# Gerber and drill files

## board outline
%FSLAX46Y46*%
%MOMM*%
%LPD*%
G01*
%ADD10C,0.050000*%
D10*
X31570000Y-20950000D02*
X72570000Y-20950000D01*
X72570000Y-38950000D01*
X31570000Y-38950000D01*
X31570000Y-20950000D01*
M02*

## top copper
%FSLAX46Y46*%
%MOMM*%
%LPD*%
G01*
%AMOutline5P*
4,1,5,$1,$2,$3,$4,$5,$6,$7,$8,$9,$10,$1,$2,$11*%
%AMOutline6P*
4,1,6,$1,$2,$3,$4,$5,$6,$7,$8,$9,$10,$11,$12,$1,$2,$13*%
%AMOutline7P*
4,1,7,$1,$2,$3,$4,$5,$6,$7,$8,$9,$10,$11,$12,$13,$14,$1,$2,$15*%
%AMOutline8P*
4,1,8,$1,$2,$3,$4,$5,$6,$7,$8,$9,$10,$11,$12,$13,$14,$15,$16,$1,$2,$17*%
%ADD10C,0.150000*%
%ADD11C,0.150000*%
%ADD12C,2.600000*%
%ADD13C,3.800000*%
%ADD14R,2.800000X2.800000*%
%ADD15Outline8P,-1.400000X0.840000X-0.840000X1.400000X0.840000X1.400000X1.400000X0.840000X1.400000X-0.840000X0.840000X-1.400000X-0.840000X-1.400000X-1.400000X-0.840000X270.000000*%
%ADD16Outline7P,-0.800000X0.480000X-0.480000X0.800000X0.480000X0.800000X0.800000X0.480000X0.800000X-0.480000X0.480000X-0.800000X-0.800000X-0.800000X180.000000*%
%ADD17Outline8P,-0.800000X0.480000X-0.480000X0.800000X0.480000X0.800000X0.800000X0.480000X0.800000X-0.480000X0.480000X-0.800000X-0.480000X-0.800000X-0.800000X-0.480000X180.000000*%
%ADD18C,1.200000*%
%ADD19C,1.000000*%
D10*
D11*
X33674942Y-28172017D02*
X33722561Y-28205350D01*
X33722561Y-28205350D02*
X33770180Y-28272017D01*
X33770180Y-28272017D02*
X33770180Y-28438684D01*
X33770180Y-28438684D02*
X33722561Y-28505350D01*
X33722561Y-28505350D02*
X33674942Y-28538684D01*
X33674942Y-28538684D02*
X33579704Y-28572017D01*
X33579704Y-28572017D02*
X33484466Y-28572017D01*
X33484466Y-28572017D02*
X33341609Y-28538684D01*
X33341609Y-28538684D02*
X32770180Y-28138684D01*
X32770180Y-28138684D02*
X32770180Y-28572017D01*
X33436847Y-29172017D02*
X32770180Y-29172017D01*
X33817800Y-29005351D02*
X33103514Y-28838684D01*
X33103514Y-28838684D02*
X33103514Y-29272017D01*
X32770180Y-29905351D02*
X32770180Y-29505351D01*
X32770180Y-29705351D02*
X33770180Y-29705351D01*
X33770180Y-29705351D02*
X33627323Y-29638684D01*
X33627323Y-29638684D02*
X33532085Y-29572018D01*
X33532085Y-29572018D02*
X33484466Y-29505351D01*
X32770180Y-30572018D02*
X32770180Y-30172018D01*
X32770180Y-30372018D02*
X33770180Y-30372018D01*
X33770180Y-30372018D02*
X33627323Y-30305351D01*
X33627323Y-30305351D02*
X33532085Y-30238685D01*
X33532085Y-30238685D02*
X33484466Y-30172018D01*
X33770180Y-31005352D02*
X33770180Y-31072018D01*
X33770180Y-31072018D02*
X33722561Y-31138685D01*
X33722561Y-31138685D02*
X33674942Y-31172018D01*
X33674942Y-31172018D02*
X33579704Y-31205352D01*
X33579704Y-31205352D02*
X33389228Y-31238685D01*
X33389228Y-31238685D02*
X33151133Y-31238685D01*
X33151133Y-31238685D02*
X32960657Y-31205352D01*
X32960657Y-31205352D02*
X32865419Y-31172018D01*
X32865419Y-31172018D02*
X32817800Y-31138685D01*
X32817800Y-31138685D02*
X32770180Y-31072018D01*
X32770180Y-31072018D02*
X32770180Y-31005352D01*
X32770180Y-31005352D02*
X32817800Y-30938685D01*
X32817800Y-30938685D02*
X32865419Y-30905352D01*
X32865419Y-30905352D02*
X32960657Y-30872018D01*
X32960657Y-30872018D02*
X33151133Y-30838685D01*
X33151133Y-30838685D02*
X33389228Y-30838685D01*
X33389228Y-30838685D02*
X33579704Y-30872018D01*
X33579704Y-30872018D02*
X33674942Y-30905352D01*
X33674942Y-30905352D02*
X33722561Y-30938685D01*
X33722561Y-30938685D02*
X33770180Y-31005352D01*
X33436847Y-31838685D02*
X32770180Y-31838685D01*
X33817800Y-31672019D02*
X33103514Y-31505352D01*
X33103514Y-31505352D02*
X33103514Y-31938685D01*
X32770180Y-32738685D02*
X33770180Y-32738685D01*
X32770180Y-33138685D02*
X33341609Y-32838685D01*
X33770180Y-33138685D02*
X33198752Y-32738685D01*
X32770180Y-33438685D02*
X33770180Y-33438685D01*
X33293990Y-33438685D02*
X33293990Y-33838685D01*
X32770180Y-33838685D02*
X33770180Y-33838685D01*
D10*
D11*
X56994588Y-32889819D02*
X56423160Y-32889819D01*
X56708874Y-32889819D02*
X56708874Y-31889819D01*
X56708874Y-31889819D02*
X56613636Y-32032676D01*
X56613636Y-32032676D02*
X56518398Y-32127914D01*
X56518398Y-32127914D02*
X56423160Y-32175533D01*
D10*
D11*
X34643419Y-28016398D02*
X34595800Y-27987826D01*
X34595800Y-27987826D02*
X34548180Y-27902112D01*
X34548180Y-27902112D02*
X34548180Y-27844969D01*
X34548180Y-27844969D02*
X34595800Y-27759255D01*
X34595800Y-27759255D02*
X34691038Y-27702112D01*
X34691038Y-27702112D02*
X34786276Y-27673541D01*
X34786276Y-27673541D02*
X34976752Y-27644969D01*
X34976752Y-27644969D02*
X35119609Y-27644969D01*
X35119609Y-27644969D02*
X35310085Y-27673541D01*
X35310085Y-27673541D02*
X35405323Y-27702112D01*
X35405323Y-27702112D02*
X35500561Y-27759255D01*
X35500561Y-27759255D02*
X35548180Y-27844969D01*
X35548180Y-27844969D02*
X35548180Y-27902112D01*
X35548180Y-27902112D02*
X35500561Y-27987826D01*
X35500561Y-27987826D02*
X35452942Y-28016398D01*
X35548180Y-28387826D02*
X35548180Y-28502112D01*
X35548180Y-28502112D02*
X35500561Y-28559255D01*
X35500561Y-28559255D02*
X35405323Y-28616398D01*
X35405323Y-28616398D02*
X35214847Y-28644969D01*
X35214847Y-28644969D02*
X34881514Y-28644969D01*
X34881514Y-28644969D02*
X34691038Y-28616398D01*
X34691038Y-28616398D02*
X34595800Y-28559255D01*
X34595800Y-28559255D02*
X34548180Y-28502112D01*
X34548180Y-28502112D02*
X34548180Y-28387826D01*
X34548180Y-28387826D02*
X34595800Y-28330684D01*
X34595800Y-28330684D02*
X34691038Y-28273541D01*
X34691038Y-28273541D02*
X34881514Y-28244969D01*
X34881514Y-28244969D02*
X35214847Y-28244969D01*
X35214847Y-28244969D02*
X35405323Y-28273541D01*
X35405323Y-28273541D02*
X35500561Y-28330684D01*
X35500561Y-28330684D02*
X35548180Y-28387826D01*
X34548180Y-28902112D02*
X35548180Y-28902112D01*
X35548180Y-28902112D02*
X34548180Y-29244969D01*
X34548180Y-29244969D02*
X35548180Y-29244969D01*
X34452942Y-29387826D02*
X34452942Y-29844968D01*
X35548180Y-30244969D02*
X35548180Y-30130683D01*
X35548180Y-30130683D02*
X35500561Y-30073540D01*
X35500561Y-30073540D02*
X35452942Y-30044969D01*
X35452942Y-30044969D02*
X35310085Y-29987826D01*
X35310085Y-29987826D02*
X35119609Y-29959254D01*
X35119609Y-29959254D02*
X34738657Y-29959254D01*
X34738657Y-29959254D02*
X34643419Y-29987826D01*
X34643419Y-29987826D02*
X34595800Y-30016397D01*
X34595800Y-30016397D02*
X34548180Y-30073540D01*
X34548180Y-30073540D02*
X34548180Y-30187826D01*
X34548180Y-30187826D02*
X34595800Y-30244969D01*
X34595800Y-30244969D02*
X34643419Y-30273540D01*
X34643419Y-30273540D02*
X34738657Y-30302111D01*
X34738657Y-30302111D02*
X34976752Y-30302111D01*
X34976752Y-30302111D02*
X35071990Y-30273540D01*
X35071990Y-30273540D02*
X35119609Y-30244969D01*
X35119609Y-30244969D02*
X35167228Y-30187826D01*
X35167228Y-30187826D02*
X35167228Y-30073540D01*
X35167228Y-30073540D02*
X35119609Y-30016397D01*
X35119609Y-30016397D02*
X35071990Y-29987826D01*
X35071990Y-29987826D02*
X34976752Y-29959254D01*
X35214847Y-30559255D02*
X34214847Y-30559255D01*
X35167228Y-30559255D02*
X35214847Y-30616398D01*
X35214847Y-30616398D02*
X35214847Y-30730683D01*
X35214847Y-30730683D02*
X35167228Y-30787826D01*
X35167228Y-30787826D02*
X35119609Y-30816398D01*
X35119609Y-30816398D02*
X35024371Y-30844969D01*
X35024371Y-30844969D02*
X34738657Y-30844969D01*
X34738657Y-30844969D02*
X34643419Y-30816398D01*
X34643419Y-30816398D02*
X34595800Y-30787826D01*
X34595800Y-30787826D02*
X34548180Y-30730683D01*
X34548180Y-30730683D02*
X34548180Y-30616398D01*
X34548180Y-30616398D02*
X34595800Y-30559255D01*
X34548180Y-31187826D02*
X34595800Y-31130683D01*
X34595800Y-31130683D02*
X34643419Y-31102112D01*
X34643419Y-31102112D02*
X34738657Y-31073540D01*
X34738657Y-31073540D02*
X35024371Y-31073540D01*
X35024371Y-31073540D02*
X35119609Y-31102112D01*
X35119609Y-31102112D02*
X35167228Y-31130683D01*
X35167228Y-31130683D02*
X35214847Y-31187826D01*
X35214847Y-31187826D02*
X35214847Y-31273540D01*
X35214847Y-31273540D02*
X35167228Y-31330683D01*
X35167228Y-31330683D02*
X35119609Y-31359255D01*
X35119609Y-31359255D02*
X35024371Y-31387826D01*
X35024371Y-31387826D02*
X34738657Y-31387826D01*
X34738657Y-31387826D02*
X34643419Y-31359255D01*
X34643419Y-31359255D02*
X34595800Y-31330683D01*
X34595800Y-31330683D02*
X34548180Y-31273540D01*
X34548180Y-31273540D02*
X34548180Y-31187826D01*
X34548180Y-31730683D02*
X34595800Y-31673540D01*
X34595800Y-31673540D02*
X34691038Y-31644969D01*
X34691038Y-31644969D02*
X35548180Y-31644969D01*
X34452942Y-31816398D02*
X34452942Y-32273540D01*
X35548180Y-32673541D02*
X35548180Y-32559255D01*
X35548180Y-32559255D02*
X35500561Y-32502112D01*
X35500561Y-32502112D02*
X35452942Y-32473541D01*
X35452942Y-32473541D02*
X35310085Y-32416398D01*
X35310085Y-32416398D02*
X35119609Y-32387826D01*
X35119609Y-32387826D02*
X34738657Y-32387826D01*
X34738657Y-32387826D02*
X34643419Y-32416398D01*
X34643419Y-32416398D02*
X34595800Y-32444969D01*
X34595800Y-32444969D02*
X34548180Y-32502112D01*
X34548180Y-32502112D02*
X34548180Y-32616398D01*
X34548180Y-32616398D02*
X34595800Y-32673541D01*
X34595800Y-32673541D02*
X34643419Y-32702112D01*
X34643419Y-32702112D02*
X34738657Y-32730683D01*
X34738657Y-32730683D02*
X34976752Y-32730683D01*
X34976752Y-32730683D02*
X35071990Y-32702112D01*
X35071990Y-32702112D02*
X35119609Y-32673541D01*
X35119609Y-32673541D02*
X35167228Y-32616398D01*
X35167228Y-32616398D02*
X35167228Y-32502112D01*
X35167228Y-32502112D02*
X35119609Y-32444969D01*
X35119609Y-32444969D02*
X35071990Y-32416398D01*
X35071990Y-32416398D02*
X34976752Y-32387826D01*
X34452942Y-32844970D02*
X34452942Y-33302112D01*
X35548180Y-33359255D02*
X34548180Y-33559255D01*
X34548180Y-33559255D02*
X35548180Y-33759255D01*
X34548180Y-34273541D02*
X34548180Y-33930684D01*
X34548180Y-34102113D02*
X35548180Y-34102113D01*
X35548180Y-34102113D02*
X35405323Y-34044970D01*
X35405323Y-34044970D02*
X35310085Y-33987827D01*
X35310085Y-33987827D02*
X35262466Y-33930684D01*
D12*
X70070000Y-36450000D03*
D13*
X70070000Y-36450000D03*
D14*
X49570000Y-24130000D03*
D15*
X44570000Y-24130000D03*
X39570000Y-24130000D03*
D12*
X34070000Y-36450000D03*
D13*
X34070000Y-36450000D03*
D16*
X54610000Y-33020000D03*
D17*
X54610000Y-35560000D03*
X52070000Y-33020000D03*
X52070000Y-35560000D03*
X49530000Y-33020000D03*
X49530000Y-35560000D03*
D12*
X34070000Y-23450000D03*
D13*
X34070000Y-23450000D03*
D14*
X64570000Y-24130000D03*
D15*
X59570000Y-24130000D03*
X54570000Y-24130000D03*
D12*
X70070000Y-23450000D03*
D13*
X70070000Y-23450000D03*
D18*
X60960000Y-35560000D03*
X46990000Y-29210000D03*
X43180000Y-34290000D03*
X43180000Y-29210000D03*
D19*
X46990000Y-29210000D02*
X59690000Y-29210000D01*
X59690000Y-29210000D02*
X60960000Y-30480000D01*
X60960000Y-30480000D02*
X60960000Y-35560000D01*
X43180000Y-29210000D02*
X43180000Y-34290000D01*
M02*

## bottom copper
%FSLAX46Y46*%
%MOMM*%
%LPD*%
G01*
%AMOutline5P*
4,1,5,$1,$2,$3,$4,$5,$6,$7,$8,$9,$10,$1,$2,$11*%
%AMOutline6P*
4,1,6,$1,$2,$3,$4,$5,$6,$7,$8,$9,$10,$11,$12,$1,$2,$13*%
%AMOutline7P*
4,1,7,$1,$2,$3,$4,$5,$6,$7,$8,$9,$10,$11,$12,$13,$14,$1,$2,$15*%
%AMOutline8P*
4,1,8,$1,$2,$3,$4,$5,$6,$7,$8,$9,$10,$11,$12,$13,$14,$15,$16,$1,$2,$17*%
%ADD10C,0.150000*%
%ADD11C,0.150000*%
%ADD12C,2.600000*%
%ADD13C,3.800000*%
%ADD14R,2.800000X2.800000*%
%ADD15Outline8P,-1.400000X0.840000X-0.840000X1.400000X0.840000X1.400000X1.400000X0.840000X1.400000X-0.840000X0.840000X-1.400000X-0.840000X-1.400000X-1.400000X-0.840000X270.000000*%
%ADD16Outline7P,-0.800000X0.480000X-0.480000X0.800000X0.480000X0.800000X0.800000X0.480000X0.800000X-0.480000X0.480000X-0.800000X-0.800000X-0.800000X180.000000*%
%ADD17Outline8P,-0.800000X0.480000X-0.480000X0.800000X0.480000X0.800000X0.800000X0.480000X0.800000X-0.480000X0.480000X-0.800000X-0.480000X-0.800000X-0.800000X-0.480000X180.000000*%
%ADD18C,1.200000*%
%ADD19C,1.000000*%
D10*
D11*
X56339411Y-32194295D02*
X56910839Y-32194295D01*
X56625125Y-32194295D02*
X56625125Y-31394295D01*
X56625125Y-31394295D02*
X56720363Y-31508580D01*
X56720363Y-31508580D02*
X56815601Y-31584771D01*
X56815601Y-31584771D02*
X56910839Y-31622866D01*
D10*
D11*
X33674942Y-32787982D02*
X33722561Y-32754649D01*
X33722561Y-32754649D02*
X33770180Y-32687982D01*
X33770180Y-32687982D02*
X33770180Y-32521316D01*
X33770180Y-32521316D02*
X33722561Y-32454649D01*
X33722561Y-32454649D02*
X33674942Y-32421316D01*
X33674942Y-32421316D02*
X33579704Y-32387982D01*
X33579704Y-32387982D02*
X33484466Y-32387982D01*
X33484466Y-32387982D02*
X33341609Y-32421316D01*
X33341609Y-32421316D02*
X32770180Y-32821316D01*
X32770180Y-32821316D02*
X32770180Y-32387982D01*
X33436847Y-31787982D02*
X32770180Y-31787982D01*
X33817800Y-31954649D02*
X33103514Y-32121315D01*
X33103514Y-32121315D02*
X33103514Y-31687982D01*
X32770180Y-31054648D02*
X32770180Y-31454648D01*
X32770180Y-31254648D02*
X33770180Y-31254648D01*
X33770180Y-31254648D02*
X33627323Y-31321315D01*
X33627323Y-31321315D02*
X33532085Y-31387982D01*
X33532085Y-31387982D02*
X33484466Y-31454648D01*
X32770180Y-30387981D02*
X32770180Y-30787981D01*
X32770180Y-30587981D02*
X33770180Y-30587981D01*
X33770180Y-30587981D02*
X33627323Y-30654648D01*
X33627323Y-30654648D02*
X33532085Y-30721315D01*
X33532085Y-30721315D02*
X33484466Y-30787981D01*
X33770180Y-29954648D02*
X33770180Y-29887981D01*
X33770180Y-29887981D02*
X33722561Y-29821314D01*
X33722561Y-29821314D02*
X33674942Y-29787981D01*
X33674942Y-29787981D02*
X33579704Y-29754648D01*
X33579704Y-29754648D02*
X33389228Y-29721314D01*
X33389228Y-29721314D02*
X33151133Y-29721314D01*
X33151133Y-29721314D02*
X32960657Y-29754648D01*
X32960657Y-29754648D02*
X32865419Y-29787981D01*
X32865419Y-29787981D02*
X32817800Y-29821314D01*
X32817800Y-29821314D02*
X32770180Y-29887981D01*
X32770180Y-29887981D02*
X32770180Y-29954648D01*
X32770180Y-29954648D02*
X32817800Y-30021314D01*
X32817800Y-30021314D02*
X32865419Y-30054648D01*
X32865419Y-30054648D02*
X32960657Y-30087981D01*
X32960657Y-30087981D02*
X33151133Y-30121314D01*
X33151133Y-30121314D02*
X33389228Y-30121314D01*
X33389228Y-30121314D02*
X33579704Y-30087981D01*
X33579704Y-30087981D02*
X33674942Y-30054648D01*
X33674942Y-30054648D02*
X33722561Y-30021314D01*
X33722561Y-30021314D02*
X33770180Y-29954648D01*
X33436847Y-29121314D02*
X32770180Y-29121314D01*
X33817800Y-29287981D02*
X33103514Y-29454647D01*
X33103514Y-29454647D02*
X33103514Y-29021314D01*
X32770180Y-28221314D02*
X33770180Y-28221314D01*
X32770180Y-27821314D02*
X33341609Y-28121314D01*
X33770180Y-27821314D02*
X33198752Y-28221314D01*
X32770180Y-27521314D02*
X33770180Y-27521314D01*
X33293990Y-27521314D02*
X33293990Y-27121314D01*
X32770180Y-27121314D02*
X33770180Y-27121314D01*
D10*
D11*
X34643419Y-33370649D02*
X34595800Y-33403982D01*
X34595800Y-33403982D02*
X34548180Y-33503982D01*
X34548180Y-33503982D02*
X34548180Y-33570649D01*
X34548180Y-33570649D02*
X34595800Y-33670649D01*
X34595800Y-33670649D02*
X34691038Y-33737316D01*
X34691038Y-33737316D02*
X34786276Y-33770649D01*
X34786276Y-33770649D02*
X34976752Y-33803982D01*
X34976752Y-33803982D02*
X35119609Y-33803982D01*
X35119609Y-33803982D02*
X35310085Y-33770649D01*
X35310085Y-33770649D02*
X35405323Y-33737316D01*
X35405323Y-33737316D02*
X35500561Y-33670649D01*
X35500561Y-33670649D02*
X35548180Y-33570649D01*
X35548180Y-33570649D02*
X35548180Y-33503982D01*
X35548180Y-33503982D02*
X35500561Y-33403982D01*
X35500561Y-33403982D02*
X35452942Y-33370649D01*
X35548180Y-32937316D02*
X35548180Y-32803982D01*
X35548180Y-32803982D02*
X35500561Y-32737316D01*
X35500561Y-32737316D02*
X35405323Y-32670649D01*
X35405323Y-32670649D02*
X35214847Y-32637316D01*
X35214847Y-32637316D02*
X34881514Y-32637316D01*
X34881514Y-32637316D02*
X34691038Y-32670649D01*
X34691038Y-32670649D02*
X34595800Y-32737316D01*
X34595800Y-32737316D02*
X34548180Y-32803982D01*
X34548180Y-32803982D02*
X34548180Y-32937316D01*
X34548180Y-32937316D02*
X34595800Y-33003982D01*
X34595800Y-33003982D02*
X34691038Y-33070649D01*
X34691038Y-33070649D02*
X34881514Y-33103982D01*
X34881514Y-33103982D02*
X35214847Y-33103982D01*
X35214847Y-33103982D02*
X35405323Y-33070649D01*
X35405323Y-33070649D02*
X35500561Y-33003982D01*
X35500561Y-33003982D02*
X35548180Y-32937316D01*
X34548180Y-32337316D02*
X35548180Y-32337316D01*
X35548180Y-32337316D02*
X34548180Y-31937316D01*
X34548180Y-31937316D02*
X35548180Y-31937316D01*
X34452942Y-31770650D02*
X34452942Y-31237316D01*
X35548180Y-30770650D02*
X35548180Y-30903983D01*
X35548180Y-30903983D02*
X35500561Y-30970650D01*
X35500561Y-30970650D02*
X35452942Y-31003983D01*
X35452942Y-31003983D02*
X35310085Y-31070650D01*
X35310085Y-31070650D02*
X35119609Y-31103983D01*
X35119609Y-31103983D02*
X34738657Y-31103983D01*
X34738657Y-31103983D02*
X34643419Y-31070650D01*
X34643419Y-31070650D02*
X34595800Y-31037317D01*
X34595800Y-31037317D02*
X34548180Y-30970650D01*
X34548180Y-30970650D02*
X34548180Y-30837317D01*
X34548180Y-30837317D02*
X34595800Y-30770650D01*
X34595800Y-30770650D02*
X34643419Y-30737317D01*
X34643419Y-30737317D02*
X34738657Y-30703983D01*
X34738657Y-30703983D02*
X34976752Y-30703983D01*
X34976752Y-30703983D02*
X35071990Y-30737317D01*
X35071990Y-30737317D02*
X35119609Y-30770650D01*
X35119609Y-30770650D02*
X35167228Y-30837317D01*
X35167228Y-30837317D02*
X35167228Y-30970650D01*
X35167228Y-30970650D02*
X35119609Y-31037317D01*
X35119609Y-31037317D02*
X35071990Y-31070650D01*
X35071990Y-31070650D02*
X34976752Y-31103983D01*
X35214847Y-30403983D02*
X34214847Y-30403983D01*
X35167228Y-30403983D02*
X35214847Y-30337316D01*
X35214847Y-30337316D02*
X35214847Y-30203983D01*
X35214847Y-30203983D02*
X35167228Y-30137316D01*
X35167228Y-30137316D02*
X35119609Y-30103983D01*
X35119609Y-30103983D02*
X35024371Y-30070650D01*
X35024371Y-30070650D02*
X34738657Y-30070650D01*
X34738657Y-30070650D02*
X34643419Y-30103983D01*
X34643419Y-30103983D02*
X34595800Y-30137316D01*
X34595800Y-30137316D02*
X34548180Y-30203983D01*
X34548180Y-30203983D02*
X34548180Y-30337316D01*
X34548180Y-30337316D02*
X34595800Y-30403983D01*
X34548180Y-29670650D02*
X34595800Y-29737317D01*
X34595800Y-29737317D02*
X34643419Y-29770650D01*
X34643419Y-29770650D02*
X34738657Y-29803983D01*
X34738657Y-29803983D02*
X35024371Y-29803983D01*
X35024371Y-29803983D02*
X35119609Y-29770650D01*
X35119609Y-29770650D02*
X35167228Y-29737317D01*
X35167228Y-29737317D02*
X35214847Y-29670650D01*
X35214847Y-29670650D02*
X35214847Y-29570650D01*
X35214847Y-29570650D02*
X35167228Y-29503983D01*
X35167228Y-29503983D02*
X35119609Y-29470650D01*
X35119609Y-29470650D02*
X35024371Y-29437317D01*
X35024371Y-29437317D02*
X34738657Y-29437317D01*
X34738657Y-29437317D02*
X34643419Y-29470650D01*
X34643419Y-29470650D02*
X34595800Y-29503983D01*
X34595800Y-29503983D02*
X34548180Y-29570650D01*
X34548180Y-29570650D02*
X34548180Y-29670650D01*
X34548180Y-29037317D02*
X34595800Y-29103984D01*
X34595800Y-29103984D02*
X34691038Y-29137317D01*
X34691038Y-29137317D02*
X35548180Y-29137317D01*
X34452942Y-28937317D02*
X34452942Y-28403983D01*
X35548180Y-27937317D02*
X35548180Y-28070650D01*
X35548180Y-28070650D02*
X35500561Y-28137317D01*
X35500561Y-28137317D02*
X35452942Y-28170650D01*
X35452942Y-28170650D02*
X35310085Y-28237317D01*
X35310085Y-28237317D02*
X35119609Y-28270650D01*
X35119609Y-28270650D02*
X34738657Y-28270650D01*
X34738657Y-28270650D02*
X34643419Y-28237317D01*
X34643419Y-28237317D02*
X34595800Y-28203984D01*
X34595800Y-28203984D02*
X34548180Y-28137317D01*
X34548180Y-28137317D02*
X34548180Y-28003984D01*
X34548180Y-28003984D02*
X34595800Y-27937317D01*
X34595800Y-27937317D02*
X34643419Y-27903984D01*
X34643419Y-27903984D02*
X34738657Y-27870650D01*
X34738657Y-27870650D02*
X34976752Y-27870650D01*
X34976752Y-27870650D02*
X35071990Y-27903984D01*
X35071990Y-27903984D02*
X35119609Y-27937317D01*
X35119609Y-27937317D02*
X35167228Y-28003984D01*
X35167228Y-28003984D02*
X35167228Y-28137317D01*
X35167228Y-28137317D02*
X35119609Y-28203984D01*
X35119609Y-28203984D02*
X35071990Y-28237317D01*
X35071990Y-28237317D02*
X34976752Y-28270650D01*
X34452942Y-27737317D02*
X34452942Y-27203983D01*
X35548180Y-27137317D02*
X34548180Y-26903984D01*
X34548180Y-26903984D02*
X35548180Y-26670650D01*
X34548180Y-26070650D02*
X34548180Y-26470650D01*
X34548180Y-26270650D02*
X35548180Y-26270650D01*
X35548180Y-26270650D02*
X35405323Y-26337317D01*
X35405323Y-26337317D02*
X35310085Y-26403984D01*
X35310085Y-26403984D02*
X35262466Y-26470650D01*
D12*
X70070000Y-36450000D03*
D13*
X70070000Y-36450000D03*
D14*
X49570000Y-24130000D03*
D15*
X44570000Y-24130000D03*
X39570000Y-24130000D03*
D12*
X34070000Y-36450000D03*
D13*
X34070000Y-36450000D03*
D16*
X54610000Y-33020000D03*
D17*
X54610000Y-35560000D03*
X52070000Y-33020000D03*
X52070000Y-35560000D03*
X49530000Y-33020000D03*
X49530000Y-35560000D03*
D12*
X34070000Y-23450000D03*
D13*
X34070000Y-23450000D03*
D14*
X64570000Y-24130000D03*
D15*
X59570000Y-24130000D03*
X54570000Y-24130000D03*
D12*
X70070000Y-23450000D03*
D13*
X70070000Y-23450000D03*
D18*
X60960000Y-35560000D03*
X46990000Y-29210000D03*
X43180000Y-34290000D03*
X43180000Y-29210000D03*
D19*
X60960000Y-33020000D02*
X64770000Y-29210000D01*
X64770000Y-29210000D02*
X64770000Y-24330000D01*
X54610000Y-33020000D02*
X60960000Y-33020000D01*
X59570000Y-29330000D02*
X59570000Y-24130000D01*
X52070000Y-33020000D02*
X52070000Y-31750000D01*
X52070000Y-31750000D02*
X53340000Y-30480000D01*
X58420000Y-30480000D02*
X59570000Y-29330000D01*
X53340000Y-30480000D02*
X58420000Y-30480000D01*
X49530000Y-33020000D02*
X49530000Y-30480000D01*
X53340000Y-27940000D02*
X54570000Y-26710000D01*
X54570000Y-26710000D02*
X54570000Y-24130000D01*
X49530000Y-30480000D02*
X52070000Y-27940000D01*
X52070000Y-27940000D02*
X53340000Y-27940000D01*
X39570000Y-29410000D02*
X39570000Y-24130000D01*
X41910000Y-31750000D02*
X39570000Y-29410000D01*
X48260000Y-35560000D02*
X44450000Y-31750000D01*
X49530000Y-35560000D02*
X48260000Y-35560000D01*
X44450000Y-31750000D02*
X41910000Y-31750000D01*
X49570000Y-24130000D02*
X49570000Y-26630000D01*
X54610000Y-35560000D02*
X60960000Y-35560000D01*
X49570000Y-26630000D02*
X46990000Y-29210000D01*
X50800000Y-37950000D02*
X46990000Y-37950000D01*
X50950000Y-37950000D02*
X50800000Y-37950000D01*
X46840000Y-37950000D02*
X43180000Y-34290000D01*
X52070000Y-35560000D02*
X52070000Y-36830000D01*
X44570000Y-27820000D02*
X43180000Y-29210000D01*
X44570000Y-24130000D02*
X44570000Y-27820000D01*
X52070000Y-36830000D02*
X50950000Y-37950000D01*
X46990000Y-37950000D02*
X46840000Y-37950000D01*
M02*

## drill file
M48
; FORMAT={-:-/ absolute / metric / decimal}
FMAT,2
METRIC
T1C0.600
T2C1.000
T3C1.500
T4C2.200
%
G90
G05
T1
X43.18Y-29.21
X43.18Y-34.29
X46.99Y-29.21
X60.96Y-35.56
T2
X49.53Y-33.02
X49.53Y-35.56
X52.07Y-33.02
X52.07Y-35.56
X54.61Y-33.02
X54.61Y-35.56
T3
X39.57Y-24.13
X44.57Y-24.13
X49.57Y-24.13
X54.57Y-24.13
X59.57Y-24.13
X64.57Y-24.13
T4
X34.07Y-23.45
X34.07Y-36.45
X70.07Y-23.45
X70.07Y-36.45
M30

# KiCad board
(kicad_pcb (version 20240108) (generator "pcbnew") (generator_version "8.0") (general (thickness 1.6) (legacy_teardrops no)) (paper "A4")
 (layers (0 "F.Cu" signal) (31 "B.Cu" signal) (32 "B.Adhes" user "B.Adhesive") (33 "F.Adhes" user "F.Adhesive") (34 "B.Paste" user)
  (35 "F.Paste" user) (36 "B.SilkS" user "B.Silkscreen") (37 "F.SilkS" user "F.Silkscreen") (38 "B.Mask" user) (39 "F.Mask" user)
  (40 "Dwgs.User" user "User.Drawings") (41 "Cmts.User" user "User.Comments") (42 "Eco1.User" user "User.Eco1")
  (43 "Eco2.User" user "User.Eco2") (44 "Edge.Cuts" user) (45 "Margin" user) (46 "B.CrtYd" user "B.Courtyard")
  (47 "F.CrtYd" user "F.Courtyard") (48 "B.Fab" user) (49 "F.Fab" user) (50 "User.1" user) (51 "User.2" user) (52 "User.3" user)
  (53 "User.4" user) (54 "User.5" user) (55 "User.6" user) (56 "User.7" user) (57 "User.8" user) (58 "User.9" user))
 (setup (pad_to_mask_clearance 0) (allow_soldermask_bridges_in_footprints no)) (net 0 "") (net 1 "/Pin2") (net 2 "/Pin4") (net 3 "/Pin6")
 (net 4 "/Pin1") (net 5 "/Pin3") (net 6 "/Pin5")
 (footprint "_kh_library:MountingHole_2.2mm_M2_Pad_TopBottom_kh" (layer "F.Cu") (at 70.07 36.45)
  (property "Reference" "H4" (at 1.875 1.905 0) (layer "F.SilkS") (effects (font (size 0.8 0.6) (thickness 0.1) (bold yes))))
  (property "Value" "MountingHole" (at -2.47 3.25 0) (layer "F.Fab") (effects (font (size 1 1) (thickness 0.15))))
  (pad "1" thru_hole circle (at 0 0) (size 2.6 2.6) (drill 2.2) (layers "*.Cu" "*.Mask") (remove_unused_layers no))
  (pad "1" connect circle (at 0 0) (size 3.8 3.8) (layers "F.Cu" "F.Mask"))
  (pad "1" connect circle (at 0 0) (size 3.8 3.8) (layers "B.Cu" "B.Mask")))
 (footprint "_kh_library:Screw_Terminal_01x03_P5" (layer "F.Cu") (at 49.57 24.13 -90)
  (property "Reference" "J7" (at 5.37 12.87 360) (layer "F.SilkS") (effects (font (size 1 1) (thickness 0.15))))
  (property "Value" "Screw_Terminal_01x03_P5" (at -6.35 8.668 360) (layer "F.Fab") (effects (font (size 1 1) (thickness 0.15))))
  (pad "1" thru_hole rect (at 0 0 270) (size 2.8 2.8) (drill 1.5) (layers "*.Cu" "*.Mask") (remove_unused_layers no) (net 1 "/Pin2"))
  (pad "2" thru_hole roundrect (at 0 5 270) (size 2.8 2.8) (drill 1.5) (layers "*.Cu" "*.Mask") (remove_unused_layers no)
   (roundrect_rratio 0) (chamfer_ratio 0.2) (chamfer top_left top_right bottom_left bottom_right) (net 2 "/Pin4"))
  (pad "3" thru_hole roundrect (at 0 10 270) (size 2.8 2.8) (drill 1.5) (layers "*.Cu" "*.Mask") (remove_unused_layers no)
   (roundrect_rratio 0) (chamfer_ratio 0.2) (chamfer top_left top_right bottom_left bottom_right) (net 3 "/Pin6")))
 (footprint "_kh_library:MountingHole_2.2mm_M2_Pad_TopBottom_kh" (layer "F.Cu") (at 34.07 36.45)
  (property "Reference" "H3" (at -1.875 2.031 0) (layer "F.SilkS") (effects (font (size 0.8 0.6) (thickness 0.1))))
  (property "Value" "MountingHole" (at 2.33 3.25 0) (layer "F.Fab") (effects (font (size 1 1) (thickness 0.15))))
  (pad "1" thru_hole circle (at 0 0) (size 2.6 2.6) (drill 2.2) (layers "*.Cu" "*.Mask") (remove_unused_layers no))
  (pad "1" connect circle (at 0 0) (size 3.8 3.8) (layers "F.Cu" "F.Mask"))
  (pad "1" connect circle (at 0 0) (size 3.8 3.8) (layers "B.Cu" "B.Mask")))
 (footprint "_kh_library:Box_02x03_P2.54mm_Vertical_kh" (layer "F.Cu") (at 54.61 33.02 180)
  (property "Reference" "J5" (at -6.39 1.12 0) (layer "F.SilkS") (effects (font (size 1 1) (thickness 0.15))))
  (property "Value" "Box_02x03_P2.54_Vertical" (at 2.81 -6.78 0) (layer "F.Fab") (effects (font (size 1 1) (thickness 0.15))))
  (pad "1" thru_hole roundrect (at 0 0 180) (size 1.6 1.6) (drill 1) (layers "*.Cu" "*.Mask") (remove_unused_layers no) (roundrect_rratio 0)
   (chamfer_ratio 0.2) (chamfer top_left top_right bottom_right) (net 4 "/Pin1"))
  (pad "2" thru_hole roundrect (at 0 -2.54 180) (size 1.6 1.6) (drill 1) (layers "*.Cu" "*.Mask") (remove_unused_layers no)
   (roundrect_rratio 0) (chamfer_ratio 0.2) (chamfer top_left top_right bottom_left bottom_right) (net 1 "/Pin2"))
  (pad "3" thru_hole roundrect (at 2.54 0 180) (size 1.6 1.6) (drill 1) (layers "*.Cu" "*.Mask") (remove_unused_layers no)
   (roundrect_rratio 0) (chamfer_ratio 0.2) (chamfer top_left top_right bottom_left bottom_right) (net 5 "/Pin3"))
  (pad "4" thru_hole roundrect (at 2.54 -2.54 180) (size 1.6 1.6) (drill 1) (layers "*.Cu" "*.Mask") (remove_unused_layers no)
   (roundrect_rratio 0) (chamfer_ratio 0.2) (chamfer top_left top_right bottom_left bottom_right) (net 2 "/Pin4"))
  (pad "5" thru_hole roundrect (at 5.08 0 180) (size 1.6 1.6) (drill 1) (layers "*.Cu" "*.Mask") (remove_unused_layers no)
   (roundrect_rratio 0) (chamfer_ratio 0.2) (chamfer top_left top_right bottom_left bottom_right) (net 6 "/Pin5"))
  (pad "6" thru_hole roundrect (at 5.08 -2.54 180) (size 1.6 1.6) (drill 1) (layers "*.Cu" "*.Mask") (remove_unused_layers no)
   (roundrect_rratio 0) (chamfer_ratio 0.2) (chamfer top_left top_right bottom_left bottom_right) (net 3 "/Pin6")))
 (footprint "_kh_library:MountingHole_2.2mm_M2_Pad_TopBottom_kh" (layer "F.Cu") (at 34.07 23.45)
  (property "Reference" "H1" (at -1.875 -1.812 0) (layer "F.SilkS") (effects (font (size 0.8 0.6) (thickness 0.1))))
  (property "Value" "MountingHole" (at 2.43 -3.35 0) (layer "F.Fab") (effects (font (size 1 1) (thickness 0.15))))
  (pad "1" thru_hole circle (at 0 0) (size 2.6 2.6) (drill 2.2) (layers "*.Cu" "*.Mask") (remove_unused_layers no))
  (pad "1" connect circle (at 0 0) (size 3.8 3.8) (layers "F.Cu" "F.Mask"))
  (pad "1" connect circle (at 0 0) (size 3.8 3.8) (layers "B.Cu" "B.Mask")))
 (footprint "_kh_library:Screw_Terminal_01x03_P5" (layer "F.Cu") (at 64.57 24.13 -90)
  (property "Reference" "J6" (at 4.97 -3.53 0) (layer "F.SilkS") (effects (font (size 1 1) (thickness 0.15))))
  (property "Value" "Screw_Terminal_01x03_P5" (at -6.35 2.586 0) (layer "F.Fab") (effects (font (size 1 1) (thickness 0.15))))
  (pad "1" thru_hole rect (at 0 0 270) (size 2.8 2.8) (drill 1.5) (layers "*.Cu" "*.Mask") (remove_unused_layers no) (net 4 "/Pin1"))
  (pad "2" thru_hole roundrect (at 0 5 270) (size 2.8 2.8) (drill 1.5) (layers "*.Cu" "*.Mask") (remove_unused_layers no)
   (roundrect_rratio 0) (chamfer_ratio 0.2) (chamfer top_left top_right bottom_left bottom_right) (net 5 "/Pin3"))
  (pad "3" thru_hole roundrect (at 0 10 270) (size 2.8 2.8) (drill 1.5) (layers "*.Cu" "*.Mask") (remove_unused_layers no)
   (roundrect_rratio 0) (chamfer_ratio 0.2) (chamfer top_left top_right bottom_left bottom_right) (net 6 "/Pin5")))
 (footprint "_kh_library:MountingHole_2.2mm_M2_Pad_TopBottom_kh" (layer "F.Cu") (at 70.07 23.45)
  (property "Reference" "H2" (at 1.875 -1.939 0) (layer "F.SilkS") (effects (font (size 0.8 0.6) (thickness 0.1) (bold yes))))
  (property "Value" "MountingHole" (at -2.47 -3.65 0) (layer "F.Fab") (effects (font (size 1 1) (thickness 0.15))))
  (pad "1" thru_hole circle (at 0 0) (size 2.6 2.6) (drill 2.2) (layers "*.Cu" "*.Mask") (remove_unused_layers no))
  (pad "1" connect circle (at 0 0) (size 3.8 3.8) (layers "F.Cu" "F.Mask"))
  (pad "1" connect circle (at 0 0) (size 3.8 3.8) (layers "B.Cu" "B.Mask")))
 (gr_rect (start 31.57 20.95) (end 72.57 38.95) (stroke (width 0.05) (type default)) (fill none) (layer "Edge.Cuts"))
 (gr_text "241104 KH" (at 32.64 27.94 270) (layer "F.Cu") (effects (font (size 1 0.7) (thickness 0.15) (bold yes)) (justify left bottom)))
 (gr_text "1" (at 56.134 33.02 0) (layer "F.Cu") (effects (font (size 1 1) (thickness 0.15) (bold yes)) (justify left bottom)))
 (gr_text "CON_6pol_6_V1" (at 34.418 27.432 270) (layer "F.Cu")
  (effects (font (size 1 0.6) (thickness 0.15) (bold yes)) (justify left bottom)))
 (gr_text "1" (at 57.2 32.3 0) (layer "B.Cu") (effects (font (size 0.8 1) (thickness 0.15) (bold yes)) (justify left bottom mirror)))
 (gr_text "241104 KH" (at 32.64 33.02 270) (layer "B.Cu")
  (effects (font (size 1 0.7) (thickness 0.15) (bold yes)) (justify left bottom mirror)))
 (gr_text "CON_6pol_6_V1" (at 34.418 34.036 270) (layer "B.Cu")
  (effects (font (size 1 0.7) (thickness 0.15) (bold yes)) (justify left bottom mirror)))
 (segment (start 60.96 33.02) (end 64.77 29.21) (width 1) (layer "B.Cu") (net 4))
 (segment (start 64.77 29.21) (end 64.77 24.33) (width 1) (layer "B.Cu") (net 4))
 (segment (start 54.61 33.02) (end 60.96 33.02) (width 1) (layer "B.Cu") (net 4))
 (segment (start 59.57 29.33) (end 59.57 24.13) (width 1) (layer "B.Cu") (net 5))
 (segment (start 52.07 33.02) (end 52.07 31.75) (width 1) (layer "B.Cu") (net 5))
 (segment (start 52.07 31.75) (end 53.34 30.48) (width 1) (layer "B.Cu") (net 5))
 (segment (start 58.42 30.48) (end 59.57 29.33) (width 1) (layer "B.Cu") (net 5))
 (segment (start 53.34 30.48) (end 58.42 30.48) (width 1) (layer "B.Cu") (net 5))
 (segment (start 49.53 33.02) (end 49.53 30.48) (width 1) (layer "B.Cu") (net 6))
 (segment (start 53.34 27.94) (end 54.57 26.71) (width 1) (layer "B.Cu") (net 6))
 (segment (start 54.57 26.71) (end 54.57 24.13) (width 1) (layer "B.Cu") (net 6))
 (segment (start 49.53 30.48) (end 52.07 27.94) (width 1) (layer "B.Cu") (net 6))
 (segment (start 52.07 27.94) (end 53.34 27.94) (width 1) (layer "B.Cu") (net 6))
 (segment (start 39.57 29.41) (end 39.57 24.13) (width 1) (layer "B.Cu") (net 3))
 (segment (start 41.91 31.75) (end 39.57 29.41) (width 1) (layer "B.Cu") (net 3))
 (segment (start 48.26 35.56) (end 44.45 31.75) (width 1) (layer "B.Cu") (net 3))
 (segment (start 49.53 35.56) (end 48.26 35.56) (width 1) (layer "B.Cu") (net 3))
 (segment (start 44.45 31.75) (end 41.91 31.75) (width 1) (layer "B.Cu") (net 3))
 (segment (start 46.99 29.21) (end 59.69 29.21) (width 1) (layer "F.Cu") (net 1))
 (segment (start 59.69 29.21) (end 60.96 30.48) (width 1) (layer "F.Cu") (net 1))
 (segment (start 60.96 30.48) (end 60.96 35.56) (width 1) (layer "F.Cu") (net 1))
 (via (at 60.96 35.56) (size 1.2) (drill 0.6) (layers "F.Cu" "B.Cu") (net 1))
 (via (at 46.99 29.21) (size 1.2) (drill 0.6) (layers "F.Cu" "B.Cu") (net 1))
 (segment (start 49.57 24.13) (end 49.57 26.63) (width 1) (layer "B.Cu") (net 1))
 (segment (start 54.61 35.56) (end 60.96 35.56) (width 1) (layer "B.Cu") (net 1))
 (segment (start 49.57 26.63) (end 46.99 29.21) (width 1) (layer "B.Cu") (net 1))
 (segment (start 43.18 29.21) (end 43.18 34.29) (width 1) (layer "F.Cu") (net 2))
 (via (at 43.18 34.29) (size 1.2) (drill 0.6) (layers "F.Cu" "B.Cu") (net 2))
 (via (at 43.18 29.21) (size 1.2) (drill 0.6) (layers "F.Cu" "B.Cu") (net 2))
 (segment (start 50.8 37.95) (end 46.99 37.95) (width 1) (layer "B.Cu") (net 2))
 (segment (start 50.95 37.95) (end 50.8 37.95) (width 1) (layer "B.Cu") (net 2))
 (segment (start 46.84 37.95) (end 43.18 34.29) (width 1) (layer "B.Cu") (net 2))
 (segment (start 52.07 35.56) (end 52.07 36.83) (width 1) (layer "B.Cu") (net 2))
 (segment (start 44.57 27.82) (end 43.18 29.21) (width 1) (layer "B.Cu") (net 2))
 (segment (start 44.57 24.13) (end 44.57 27.82) (width 1) (layer "B.Cu") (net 2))
 (segment (start 52.07 36.83) (end 50.95 37.95) (width 1) (layer "B.Cu") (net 2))
 (segment (start 46.99 37.95) (end 46.84 37.95) (width 1) (layer "B.Cu") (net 2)))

